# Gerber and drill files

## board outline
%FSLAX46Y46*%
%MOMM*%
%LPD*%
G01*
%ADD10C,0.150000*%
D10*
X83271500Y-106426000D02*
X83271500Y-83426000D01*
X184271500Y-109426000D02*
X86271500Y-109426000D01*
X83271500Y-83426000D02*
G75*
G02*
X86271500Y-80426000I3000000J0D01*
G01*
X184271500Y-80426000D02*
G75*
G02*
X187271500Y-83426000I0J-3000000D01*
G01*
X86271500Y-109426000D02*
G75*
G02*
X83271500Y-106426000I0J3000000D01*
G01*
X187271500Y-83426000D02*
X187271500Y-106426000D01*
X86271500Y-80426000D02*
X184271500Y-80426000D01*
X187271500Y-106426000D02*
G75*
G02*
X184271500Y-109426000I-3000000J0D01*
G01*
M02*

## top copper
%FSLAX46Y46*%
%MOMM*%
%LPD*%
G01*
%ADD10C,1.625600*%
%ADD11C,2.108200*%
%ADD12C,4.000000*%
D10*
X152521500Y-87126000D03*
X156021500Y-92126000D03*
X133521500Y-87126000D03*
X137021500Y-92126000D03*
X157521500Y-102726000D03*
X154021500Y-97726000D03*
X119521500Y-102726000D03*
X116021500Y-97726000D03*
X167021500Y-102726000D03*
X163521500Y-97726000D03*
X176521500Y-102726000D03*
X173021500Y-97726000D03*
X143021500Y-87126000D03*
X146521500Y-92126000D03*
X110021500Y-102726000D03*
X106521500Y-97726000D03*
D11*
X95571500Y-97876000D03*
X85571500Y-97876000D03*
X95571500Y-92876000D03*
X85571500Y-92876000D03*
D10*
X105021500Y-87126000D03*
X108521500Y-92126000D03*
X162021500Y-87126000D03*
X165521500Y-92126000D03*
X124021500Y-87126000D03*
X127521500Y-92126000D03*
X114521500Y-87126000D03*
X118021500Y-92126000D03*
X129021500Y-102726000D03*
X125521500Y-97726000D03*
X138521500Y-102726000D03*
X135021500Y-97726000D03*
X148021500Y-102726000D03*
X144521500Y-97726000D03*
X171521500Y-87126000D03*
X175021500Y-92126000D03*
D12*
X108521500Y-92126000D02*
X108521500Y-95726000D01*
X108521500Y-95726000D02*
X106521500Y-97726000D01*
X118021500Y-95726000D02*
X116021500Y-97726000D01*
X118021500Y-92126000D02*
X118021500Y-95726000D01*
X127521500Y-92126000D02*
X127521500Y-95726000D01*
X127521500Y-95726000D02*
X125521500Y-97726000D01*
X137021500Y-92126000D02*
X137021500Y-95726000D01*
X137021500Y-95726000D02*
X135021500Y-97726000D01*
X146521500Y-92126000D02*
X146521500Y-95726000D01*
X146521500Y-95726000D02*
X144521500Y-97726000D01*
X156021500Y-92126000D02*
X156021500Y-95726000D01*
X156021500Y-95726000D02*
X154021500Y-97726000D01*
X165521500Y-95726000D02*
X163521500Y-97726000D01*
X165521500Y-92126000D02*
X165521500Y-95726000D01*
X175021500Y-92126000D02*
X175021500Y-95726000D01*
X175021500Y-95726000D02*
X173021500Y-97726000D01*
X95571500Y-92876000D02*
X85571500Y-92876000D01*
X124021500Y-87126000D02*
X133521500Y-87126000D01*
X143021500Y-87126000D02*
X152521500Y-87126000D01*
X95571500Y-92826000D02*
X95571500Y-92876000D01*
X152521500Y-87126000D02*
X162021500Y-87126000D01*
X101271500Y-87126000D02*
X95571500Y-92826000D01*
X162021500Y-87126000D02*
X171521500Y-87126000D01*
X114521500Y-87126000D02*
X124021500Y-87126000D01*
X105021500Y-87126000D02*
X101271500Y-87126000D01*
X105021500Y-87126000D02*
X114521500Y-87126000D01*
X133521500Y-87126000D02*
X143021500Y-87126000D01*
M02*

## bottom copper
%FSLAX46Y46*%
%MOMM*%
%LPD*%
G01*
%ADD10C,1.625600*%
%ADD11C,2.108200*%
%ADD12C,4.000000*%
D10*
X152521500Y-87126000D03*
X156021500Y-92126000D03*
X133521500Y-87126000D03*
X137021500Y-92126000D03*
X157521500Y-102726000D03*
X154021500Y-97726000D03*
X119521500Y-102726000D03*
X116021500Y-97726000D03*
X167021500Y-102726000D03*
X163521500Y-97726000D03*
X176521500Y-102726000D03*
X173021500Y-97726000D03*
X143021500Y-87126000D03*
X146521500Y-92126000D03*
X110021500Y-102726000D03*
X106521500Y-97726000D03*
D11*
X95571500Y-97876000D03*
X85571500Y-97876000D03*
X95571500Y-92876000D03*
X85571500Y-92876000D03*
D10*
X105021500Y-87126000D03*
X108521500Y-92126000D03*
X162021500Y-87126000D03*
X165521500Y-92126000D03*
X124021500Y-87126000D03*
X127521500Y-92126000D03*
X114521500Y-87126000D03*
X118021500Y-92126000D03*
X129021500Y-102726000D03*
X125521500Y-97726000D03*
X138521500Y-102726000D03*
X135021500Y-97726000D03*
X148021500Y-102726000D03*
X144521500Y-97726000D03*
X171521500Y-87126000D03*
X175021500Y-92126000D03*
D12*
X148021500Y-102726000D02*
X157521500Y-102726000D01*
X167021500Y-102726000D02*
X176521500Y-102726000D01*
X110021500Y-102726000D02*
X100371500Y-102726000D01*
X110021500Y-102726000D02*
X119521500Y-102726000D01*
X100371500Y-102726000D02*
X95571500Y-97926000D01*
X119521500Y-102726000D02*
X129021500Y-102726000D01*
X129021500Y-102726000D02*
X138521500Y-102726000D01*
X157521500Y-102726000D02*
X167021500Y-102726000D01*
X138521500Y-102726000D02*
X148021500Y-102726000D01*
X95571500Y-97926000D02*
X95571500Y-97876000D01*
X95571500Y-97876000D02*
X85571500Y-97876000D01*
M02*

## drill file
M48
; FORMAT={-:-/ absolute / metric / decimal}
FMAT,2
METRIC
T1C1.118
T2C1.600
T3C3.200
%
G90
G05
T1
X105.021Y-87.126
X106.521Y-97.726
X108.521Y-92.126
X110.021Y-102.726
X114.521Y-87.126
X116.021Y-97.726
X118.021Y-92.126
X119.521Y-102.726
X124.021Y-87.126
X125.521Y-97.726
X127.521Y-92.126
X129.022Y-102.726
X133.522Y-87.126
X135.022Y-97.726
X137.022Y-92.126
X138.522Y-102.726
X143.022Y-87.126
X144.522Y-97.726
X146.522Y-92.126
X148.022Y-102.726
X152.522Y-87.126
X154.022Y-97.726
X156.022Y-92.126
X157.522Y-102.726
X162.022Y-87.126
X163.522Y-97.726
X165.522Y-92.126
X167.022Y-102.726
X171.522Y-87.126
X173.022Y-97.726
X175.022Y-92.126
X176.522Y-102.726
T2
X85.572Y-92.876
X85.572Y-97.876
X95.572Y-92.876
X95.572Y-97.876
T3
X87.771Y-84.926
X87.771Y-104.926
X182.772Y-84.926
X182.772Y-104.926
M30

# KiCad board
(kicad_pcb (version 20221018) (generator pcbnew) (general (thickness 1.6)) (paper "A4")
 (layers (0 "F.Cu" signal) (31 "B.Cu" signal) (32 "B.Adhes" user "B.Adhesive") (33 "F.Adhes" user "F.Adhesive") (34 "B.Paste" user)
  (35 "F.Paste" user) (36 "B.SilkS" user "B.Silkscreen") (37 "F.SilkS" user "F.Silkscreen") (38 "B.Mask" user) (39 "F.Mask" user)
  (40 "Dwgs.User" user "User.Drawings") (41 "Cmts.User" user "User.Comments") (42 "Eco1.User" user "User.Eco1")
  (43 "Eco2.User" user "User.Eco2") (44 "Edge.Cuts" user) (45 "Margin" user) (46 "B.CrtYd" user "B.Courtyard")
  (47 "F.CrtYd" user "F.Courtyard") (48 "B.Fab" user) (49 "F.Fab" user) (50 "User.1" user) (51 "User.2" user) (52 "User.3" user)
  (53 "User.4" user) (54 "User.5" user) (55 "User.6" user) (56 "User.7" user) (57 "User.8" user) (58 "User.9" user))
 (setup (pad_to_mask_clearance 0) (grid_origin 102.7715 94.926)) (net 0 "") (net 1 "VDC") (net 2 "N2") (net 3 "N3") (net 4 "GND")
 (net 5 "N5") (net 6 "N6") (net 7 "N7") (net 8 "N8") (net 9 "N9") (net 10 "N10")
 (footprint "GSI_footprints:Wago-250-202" (layer "F.Cu") (at 152.5215 87.126 180)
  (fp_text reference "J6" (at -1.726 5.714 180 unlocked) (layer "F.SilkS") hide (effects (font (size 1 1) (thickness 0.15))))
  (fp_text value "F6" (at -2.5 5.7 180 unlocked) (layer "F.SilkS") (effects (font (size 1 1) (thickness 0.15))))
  (pad "1" thru_hole circle (at 0 0 180) (size 1.6256 1.6256) (drill 1.1176) (layers "*.Cu" "*.Mask") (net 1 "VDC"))
  (pad "2" thru_hole circle (at -3.5 -5 180) (size 1.6256 1.6256) (drill 1.1176) (layers "*.Cu" "*.Mask") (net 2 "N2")))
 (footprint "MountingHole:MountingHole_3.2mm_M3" (layer "F.Cu") (at 182.7715 104.926)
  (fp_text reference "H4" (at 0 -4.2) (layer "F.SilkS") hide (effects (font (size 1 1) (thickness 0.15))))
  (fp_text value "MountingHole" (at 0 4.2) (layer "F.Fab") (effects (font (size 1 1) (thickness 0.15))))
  (pad "" np_thru_hole circle (at 0 0) (size 3.2 3.2) (drill 3.2) (layers "*.Cu" "*.Mask")))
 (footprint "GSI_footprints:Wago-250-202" (layer "F.Cu") (at 133.5215 87.126 180)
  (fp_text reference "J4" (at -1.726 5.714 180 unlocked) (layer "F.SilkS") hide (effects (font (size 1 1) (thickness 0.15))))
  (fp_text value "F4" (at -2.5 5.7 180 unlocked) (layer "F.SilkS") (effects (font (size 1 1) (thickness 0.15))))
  (pad "1" thru_hole circle (at 0 0 180) (size 1.6256 1.6256) (drill 1.1176) (layers "*.Cu" "*.Mask") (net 1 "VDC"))
  (pad "2" thru_hole circle (at -3.5 -5 180) (size 1.6256 1.6256) (drill 1.1176) (layers "*.Cu" "*.Mask") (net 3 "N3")))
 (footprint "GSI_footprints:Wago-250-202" (layer "F.Cu") (at 157.5215 102.726)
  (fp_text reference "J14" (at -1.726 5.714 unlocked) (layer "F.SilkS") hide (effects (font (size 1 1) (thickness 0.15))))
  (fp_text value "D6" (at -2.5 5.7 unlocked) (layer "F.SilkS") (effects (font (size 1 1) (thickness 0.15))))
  (pad "1" thru_hole circle (at 0 0) (size 1.6256 1.6256) (drill 1.1176) (layers "*.Cu" "*.Mask") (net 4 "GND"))
  (pad "2" thru_hole circle (at -3.5 -5) (size 1.6256 1.6256) (drill 1.1176) (layers "*.Cu" "*.Mask") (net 2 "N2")))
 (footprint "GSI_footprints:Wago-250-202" (layer "F.Cu") (at 119.5215 102.726)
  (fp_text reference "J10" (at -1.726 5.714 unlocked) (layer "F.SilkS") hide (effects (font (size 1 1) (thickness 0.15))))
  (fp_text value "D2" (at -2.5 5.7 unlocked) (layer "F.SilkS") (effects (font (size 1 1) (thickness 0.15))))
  (pad "1" thru_hole circle (at 0 0) (size 1.6256 1.6256) (drill 1.1176) (layers "*.Cu" "*.Mask") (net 4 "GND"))
  (pad "2" thru_hole circle (at -3.5 -5) (size 1.6256 1.6256) (drill 1.1176) (layers "*.Cu" "*.Mask") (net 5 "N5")))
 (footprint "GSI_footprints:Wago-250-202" (layer "F.Cu") (at 167.0215 102.726)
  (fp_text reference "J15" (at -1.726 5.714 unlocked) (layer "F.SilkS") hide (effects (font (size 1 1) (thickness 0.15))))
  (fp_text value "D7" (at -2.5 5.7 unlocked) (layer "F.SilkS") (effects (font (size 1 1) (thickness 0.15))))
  (pad "1" thru_hole circle (at 0 0) (size 1.6256 1.6256) (drill 1.1176) (layers "*.Cu" "*.Mask") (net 4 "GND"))
  (pad "2" thru_hole circle (at -3.5 -5) (size 1.6256 1.6256) (drill 1.1176) (layers "*.Cu" "*.Mask") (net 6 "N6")))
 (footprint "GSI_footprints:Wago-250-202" (layer "F.Cu") (at 176.5215 102.726)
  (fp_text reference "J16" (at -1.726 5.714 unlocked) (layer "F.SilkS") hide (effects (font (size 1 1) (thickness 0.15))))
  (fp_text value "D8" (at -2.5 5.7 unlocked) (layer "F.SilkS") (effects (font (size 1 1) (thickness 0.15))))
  (pad "1" thru_hole circle (at 0 0) (size 1.6256 1.6256) (drill 1.1176) (layers "*.Cu" "*.Mask") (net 4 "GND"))
  (pad "2" thru_hole circle (at -3.5 -5) (size 1.6256 1.6256) (drill 1.1176) (layers "*.Cu" "*.Mask") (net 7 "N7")))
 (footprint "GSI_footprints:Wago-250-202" (layer "F.Cu") (at 143.0215 87.126 180)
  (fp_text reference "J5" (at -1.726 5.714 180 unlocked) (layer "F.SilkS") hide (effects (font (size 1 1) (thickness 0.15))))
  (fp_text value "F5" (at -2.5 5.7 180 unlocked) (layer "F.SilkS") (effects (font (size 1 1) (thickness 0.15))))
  (pad "1" thru_hole circle (at 0 0 180) (size 1.6256 1.6256) (drill 1.1176) (layers "*.Cu" "*.Mask") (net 1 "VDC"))
  (pad "2" thru_hole circle (at -3.5 -5 180) (size 1.6256 1.6256) (drill 1.1176) (layers "*.Cu" "*.Mask") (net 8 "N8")))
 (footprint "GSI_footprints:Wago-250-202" (layer "F.Cu") (at 110.0215 102.726)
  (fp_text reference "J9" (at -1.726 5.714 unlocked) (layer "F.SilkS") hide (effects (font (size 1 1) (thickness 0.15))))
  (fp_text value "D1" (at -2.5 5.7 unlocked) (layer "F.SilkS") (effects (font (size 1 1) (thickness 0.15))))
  (pad "1" thru_hole circle (at 0 0) (size 1.6256 1.6256) (drill 1.1176) (layers "*.Cu" "*.Mask") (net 4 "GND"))
  (pad "2" thru_hole circle (at -3.5 -5) (size 1.6256 1.6256) (drill 1.1176) (layers "*.Cu" "*.Mask") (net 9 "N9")))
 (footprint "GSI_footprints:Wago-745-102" (layer "F.Cu") (at 85.5715 97.876 -90)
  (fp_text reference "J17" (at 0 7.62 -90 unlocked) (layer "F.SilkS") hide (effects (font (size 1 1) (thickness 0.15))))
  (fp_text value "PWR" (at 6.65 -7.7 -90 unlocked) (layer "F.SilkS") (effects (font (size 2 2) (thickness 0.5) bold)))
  (pad "1" thru_hole circle (at 0 -10 270) (size 2.1082 2.1082) (drill 1.6002) (layers "*.Cu" "*.Mask") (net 4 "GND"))
  (pad "1" thru_hole circle (at 0 0 270) (size 2.1082 2.1082) (drill 1.6002) (layers "*.Cu" "*.Mask") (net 4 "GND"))
  (pad "2" thru_hole circle (at -5 -10 270) (size 2.1082 2.1082) (drill 1.6002) (layers "*.Cu" "*.Mask") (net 1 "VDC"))
  (pad "2" thru_hole circle (at -5 0 270) (size 2.1082 2.1082) (drill 1.6002) (layers "*.Cu" "*.Mask") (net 1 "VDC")))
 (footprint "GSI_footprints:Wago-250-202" (layer "F.Cu") (at 105.0215 87.126 180)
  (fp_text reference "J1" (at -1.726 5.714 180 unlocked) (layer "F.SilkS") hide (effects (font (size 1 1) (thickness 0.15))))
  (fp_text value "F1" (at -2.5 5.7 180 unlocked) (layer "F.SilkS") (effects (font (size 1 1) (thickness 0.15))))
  (pad "1" thru_hole circle (at 0 0 180) (size 1.6256 1.6256) (drill 1.1176) (layers "*.Cu" "*.Mask") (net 1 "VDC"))
  (pad "2" thru_hole circle (at -3.5 -5 180) (size 1.6256 1.6256) (drill 1.1176) (layers "*.Cu" "*.Mask") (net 9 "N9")))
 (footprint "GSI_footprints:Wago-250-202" (layer "F.Cu") (at 162.0215 87.126 180)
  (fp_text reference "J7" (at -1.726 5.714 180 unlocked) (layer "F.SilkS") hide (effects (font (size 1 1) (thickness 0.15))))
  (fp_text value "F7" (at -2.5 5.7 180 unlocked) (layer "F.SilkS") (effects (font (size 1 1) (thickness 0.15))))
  (pad "1" thru_hole circle (at 0 0 180) (size 1.6256 1.6256) (drill 1.1176) (layers "*.Cu" "*.Mask") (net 1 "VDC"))
  (pad "2" thru_hole circle (at -3.5 -5 180) (size 1.6256 1.6256) (drill 1.1176) (layers "*.Cu" "*.Mask") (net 6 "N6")))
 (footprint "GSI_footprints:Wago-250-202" (layer "F.Cu") (at 124.0215 87.126 180)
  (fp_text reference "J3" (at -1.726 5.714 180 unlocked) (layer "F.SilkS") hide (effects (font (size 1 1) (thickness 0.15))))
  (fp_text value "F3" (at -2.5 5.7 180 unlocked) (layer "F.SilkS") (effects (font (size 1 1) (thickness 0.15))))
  (pad "1" thru_hole circle (at 0 0 180) (size 1.6256 1.6256) (drill 1.1176) (layers "*.Cu" "*.Mask") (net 1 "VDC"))
  (pad "2" thru_hole circle (at -3.5 -5 180) (size 1.6256 1.6256) (drill 1.1176) (layers "*.Cu" "*.Mask") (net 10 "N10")))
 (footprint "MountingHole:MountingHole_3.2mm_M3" (layer "F.Cu") (at 182.7715 84.926)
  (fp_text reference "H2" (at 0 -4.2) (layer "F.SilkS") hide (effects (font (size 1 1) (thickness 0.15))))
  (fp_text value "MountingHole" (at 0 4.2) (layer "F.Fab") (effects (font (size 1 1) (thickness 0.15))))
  (pad "" np_thru_hole circle (at 0 0) (size 3.2 3.2) (drill 3.2) (layers "*.Cu" "*.Mask")))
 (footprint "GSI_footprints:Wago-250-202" (layer "F.Cu") (at 114.5215 87.126 180)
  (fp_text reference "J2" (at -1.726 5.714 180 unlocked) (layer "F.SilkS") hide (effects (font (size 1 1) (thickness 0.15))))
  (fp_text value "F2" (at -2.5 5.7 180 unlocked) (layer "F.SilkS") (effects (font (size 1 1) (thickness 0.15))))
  (pad "1" thru_hole circle (at 0 0 180) (size 1.6256 1.6256) (drill 1.1176) (layers "*.Cu" "*.Mask") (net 1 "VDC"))
  (pad "2" thru_hole circle (at -3.5 -5 180) (size 1.6256 1.6256) (drill 1.1176) (layers "*.Cu" "*.Mask") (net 5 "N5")))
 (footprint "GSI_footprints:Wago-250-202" (layer "F.Cu") (at 129.0215 102.726)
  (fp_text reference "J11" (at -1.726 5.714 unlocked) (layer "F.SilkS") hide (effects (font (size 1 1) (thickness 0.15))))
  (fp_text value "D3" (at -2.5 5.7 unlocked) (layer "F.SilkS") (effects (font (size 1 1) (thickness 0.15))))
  (pad "1" thru_hole circle (at 0 0) (size 1.6256 1.6256) (drill 1.1176) (layers "*.Cu" "*.Mask") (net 4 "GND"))
  (pad "2" thru_hole circle (at -3.5 -5) (size 1.6256 1.6256) (drill 1.1176) (layers "*.Cu" "*.Mask") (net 10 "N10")))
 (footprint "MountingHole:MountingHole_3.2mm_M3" (layer "F.Cu") (at 87.7715 104.926)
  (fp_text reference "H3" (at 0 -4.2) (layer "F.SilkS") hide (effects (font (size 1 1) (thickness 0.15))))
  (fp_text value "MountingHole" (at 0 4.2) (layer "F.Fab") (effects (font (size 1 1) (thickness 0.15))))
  (pad "" np_thru_hole circle (at 0 0) (size 3.2 3.2) (drill 3.2) (layers "*.Cu" "*.Mask")))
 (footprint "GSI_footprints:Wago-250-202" (layer "F.Cu") (at 138.5215 102.726)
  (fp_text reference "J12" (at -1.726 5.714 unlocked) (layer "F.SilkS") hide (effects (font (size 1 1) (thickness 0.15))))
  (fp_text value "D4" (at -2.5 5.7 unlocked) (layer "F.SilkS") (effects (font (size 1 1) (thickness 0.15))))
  (pad "1" thru_hole circle (at 0 0) (size 1.6256 1.6256) (drill 1.1176) (layers "*.Cu" "*.Mask") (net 4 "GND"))
  (pad "2" thru_hole circle (at -3.5 -5) (size 1.6256 1.6256) (drill 1.1176) (layers "*.Cu" "*.Mask") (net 3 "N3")))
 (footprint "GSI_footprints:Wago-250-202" (layer "F.Cu") (at 148.0215 102.726)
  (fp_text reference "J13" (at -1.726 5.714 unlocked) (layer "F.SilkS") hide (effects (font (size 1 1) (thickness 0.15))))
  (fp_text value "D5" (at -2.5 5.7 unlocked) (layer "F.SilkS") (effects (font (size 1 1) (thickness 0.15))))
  (pad "1" thru_hole circle (at 0 0) (size 1.6256 1.6256) (drill 1.1176) (layers "*.Cu" "*.Mask") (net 4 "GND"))
  (pad "2" thru_hole circle (at -3.5 -5) (size 1.6256 1.6256) (drill 1.1176) (layers "*.Cu" "*.Mask") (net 8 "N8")))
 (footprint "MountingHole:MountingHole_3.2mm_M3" (layer "F.Cu") (at 87.7715 84.926)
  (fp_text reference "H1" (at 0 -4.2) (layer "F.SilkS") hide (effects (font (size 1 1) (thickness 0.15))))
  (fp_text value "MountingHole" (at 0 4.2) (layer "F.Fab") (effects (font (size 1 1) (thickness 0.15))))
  (pad "" np_thru_hole circle (at 0 0) (size 3.2 3.2) (drill 3.2) (layers "*.Cu" "*.Mask")))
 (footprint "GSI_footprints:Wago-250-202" (layer "F.Cu") (at 171.5215 87.126 180)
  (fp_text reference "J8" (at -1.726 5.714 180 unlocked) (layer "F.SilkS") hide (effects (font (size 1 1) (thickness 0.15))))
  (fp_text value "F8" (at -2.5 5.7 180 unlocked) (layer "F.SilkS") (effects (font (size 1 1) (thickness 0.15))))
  (pad "1" thru_hole circle (at 0 0 180) (size 1.6256 1.6256) (drill 1.1176) (layers "*.Cu" "*.Mask") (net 1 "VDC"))
  (pad "2" thru_hole circle (at -3.5 -5 180) (size 1.6256 1.6256) (drill 1.1176) (layers "*.Cu" "*.Mask") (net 7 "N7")))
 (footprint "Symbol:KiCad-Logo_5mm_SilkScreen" (layer "B.Cu") (at 98.3715 105.126 180)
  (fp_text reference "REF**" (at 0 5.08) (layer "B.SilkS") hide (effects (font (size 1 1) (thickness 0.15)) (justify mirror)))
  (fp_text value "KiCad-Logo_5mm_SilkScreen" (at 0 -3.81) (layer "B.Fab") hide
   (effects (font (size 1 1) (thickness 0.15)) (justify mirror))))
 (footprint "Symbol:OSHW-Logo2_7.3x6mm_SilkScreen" (layer "B.Cu") (at 172.0715 104.926 180)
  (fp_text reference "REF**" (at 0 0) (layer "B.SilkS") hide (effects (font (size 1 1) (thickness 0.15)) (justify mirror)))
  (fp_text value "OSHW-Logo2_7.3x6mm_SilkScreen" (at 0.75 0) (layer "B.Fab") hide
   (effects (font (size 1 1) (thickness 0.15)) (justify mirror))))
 (gr_line (start 83.2715 106.426) (end 83.2715 83.426) (stroke (width 0.15) (type default)) (layer "Edge.Cuts"))
 (gr_line (start 184.2715 109.426) (end 86.2715 109.426) (stroke (width 0.15) (type default)) (layer "Edge.Cuts"))
 (gr_arc (start 83.2715 83.426) (mid 84.15018 81.30468) (end 86.2715 80.426) (stroke (width 0.15) (type default)) (layer "Edge.Cuts"))
 (gr_arc (start 184.2715 80.426) (mid 186.39282 81.30468) (end 187.2715 83.426) (stroke (width 0.15) (type default)) (layer "Edge.Cuts"))
 (gr_arc (start 86.2715 109.426) (mid 84.15018 108.54732) (end 83.2715 106.426) (stroke (width 0.15) (type default)) (layer "Edge.Cuts"))
 (gr_line (start 187.2715 83.426) (end 187.2715 106.426) (stroke (width 0.15) (type default)) (layer "Edge.Cuts"))
 (gr_line (start 86.2715 80.426) (end 184.2715 80.426) (stroke (width 0.15) (type default)) (layer "Edge.Cuts"))
 (gr_arc (start 187.2715 106.426) (mid 186.39282 108.54732) (end 184.2715 109.426) (stroke (width 0.15) (type default)) (layer "Edge.Cuts"))
 (segment (start 108.5215 92.126) (end 108.5215 95.726) (width 4) (layer "F.Cu") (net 9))
 (segment (start 108.5215 95.726) (end 106.5215 97.726) (width 4) (layer "F.Cu") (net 9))
 (segment (start 118.0215 95.726) (end 116.0215 97.726) (width 4) (layer "F.Cu") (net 5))
 (segment (start 118.0215 92.126) (end 118.0215 95.726) (width 4) (layer "F.Cu") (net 5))
 (segment (start 127.5215 92.126) (end 127.5215 95.726) (width 4) (layer "F.Cu") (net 10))
 (segment (start 127.5215 95.726) (end 125.5215 97.726) (width 4) (layer "F.Cu") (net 10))
 (segment (start 137.0215 92.126) (end 137.0215 95.726) (width 4) (layer "F.Cu") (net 3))
 (segment (start 137.0215 95.726) (end 135.0215 97.726) (width 4) (layer "F.Cu") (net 3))
 (segment (start 146.5215 92.126) (end 146.5215 95.726) (width 4) (layer "F.Cu") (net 8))
 (segment (start 146.5215 95.726) (end 144.5215 97.726) (width 4) (layer "F.Cu") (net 8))
 (segment (start 156.0215 92.126) (end 156.0215 95.726) (width 4) (layer "F.Cu") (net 2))
 (segment (start 156.0215 95.726) (end 154.0215 97.726) (width 4) (layer "F.Cu") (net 2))
 (segment (start 165.5215 95.726) (end 163.5215 97.726) (width 4) (layer "F.Cu") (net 6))
 (segment (start 165.5215 92.126) (end 165.5215 95.726) (width 4) (layer "F.Cu") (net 6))
 (segment (start 175.0215 92.126) (end 175.0215 95.726) (width 4) (layer "F.Cu") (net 7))
 (segment (start 175.0215 95.726) (end 173.0215 97.726) (width 4) (layer "F.Cu") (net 7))
 (segment (start 95.5715 92.876) (end 85.5715 92.876) (width 4) (layer "F.Cu") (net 1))
 (segment (start 124.0215 87.126) (end 133.5215 87.126) (width 4) (layer "F.Cu") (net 1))
 (segment (start 143.0215 87.126) (end 152.5215 87.126) (width 4) (layer "F.Cu") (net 1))
 (segment (start 95.5715 92.826) (end 95.5715 92.876) (width 4) (layer "F.Cu") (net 1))
 (segment (start 152.5215 87.126) (end 162.0215 87.126) (width 4) (layer "F.Cu") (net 1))
 (segment (start 101.2715 87.126) (end 95.5715 92.826) (width 4) (layer "F.Cu") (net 1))
 (segment (start 162.0215 87.126) (end 171.5215 87.126) (width 4) (layer "F.Cu") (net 1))
 (segment (start 114.5215 87.126) (end 124.0215 87.126) (width 4) (layer "F.Cu") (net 1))
 (segment (start 105.0215 87.126) (end 101.2715 87.126) (width 4) (layer "F.Cu") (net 1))
 (segment (start 105.0215 87.126) (end 114.5215 87.126) (width 4) (layer "F.Cu") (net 1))
 (segment (start 133.5215 87.126) (end 143.0215 87.126) (width 4) (layer "F.Cu") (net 1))
 (segment (start 148.0215 102.726) (end 157.5215 102.726) (width 4) (layer "B.Cu") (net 4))
 (segment (start 167.0215 102.726) (end 176.5215 102.726) (width 4) (layer "B.Cu") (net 4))
 (segment (start 110.0215 102.726) (end 100.3715 102.726) (width 4) (layer "B.Cu") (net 4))
 (segment (start 110.0215 102.726) (end 119.5215 102.726) (width 4) (layer "B.Cu") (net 4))
 (segment (start 100.3715 102.726) (end 95.5715 97.926) (width 4) (layer "B.Cu") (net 4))
 (segment (start 119.5215 102.726) (end 129.0215 102.726) (width 4) (layer "B.Cu") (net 4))
 (segment (start 129.0215 102.726) (end 138.5215 102.726) (width 4) (layer "B.Cu") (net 4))
 (segment (start 157.5215 102.726) (end 167.0215 102.726) (width 4) (layer "B.Cu") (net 4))
 (segment (start 138.5215 102.726) (end 148.0215 102.726) (width 4) (layer "B.Cu") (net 4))
 (segment (start 95.5715 97.926) (end 95.5715 97.876) (width 4) (layer "B.Cu") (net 4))
 (segment (start 95.5715 97.876) (end 85.5715 97.876) (width 4) (layer "B.Cu") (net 4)))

